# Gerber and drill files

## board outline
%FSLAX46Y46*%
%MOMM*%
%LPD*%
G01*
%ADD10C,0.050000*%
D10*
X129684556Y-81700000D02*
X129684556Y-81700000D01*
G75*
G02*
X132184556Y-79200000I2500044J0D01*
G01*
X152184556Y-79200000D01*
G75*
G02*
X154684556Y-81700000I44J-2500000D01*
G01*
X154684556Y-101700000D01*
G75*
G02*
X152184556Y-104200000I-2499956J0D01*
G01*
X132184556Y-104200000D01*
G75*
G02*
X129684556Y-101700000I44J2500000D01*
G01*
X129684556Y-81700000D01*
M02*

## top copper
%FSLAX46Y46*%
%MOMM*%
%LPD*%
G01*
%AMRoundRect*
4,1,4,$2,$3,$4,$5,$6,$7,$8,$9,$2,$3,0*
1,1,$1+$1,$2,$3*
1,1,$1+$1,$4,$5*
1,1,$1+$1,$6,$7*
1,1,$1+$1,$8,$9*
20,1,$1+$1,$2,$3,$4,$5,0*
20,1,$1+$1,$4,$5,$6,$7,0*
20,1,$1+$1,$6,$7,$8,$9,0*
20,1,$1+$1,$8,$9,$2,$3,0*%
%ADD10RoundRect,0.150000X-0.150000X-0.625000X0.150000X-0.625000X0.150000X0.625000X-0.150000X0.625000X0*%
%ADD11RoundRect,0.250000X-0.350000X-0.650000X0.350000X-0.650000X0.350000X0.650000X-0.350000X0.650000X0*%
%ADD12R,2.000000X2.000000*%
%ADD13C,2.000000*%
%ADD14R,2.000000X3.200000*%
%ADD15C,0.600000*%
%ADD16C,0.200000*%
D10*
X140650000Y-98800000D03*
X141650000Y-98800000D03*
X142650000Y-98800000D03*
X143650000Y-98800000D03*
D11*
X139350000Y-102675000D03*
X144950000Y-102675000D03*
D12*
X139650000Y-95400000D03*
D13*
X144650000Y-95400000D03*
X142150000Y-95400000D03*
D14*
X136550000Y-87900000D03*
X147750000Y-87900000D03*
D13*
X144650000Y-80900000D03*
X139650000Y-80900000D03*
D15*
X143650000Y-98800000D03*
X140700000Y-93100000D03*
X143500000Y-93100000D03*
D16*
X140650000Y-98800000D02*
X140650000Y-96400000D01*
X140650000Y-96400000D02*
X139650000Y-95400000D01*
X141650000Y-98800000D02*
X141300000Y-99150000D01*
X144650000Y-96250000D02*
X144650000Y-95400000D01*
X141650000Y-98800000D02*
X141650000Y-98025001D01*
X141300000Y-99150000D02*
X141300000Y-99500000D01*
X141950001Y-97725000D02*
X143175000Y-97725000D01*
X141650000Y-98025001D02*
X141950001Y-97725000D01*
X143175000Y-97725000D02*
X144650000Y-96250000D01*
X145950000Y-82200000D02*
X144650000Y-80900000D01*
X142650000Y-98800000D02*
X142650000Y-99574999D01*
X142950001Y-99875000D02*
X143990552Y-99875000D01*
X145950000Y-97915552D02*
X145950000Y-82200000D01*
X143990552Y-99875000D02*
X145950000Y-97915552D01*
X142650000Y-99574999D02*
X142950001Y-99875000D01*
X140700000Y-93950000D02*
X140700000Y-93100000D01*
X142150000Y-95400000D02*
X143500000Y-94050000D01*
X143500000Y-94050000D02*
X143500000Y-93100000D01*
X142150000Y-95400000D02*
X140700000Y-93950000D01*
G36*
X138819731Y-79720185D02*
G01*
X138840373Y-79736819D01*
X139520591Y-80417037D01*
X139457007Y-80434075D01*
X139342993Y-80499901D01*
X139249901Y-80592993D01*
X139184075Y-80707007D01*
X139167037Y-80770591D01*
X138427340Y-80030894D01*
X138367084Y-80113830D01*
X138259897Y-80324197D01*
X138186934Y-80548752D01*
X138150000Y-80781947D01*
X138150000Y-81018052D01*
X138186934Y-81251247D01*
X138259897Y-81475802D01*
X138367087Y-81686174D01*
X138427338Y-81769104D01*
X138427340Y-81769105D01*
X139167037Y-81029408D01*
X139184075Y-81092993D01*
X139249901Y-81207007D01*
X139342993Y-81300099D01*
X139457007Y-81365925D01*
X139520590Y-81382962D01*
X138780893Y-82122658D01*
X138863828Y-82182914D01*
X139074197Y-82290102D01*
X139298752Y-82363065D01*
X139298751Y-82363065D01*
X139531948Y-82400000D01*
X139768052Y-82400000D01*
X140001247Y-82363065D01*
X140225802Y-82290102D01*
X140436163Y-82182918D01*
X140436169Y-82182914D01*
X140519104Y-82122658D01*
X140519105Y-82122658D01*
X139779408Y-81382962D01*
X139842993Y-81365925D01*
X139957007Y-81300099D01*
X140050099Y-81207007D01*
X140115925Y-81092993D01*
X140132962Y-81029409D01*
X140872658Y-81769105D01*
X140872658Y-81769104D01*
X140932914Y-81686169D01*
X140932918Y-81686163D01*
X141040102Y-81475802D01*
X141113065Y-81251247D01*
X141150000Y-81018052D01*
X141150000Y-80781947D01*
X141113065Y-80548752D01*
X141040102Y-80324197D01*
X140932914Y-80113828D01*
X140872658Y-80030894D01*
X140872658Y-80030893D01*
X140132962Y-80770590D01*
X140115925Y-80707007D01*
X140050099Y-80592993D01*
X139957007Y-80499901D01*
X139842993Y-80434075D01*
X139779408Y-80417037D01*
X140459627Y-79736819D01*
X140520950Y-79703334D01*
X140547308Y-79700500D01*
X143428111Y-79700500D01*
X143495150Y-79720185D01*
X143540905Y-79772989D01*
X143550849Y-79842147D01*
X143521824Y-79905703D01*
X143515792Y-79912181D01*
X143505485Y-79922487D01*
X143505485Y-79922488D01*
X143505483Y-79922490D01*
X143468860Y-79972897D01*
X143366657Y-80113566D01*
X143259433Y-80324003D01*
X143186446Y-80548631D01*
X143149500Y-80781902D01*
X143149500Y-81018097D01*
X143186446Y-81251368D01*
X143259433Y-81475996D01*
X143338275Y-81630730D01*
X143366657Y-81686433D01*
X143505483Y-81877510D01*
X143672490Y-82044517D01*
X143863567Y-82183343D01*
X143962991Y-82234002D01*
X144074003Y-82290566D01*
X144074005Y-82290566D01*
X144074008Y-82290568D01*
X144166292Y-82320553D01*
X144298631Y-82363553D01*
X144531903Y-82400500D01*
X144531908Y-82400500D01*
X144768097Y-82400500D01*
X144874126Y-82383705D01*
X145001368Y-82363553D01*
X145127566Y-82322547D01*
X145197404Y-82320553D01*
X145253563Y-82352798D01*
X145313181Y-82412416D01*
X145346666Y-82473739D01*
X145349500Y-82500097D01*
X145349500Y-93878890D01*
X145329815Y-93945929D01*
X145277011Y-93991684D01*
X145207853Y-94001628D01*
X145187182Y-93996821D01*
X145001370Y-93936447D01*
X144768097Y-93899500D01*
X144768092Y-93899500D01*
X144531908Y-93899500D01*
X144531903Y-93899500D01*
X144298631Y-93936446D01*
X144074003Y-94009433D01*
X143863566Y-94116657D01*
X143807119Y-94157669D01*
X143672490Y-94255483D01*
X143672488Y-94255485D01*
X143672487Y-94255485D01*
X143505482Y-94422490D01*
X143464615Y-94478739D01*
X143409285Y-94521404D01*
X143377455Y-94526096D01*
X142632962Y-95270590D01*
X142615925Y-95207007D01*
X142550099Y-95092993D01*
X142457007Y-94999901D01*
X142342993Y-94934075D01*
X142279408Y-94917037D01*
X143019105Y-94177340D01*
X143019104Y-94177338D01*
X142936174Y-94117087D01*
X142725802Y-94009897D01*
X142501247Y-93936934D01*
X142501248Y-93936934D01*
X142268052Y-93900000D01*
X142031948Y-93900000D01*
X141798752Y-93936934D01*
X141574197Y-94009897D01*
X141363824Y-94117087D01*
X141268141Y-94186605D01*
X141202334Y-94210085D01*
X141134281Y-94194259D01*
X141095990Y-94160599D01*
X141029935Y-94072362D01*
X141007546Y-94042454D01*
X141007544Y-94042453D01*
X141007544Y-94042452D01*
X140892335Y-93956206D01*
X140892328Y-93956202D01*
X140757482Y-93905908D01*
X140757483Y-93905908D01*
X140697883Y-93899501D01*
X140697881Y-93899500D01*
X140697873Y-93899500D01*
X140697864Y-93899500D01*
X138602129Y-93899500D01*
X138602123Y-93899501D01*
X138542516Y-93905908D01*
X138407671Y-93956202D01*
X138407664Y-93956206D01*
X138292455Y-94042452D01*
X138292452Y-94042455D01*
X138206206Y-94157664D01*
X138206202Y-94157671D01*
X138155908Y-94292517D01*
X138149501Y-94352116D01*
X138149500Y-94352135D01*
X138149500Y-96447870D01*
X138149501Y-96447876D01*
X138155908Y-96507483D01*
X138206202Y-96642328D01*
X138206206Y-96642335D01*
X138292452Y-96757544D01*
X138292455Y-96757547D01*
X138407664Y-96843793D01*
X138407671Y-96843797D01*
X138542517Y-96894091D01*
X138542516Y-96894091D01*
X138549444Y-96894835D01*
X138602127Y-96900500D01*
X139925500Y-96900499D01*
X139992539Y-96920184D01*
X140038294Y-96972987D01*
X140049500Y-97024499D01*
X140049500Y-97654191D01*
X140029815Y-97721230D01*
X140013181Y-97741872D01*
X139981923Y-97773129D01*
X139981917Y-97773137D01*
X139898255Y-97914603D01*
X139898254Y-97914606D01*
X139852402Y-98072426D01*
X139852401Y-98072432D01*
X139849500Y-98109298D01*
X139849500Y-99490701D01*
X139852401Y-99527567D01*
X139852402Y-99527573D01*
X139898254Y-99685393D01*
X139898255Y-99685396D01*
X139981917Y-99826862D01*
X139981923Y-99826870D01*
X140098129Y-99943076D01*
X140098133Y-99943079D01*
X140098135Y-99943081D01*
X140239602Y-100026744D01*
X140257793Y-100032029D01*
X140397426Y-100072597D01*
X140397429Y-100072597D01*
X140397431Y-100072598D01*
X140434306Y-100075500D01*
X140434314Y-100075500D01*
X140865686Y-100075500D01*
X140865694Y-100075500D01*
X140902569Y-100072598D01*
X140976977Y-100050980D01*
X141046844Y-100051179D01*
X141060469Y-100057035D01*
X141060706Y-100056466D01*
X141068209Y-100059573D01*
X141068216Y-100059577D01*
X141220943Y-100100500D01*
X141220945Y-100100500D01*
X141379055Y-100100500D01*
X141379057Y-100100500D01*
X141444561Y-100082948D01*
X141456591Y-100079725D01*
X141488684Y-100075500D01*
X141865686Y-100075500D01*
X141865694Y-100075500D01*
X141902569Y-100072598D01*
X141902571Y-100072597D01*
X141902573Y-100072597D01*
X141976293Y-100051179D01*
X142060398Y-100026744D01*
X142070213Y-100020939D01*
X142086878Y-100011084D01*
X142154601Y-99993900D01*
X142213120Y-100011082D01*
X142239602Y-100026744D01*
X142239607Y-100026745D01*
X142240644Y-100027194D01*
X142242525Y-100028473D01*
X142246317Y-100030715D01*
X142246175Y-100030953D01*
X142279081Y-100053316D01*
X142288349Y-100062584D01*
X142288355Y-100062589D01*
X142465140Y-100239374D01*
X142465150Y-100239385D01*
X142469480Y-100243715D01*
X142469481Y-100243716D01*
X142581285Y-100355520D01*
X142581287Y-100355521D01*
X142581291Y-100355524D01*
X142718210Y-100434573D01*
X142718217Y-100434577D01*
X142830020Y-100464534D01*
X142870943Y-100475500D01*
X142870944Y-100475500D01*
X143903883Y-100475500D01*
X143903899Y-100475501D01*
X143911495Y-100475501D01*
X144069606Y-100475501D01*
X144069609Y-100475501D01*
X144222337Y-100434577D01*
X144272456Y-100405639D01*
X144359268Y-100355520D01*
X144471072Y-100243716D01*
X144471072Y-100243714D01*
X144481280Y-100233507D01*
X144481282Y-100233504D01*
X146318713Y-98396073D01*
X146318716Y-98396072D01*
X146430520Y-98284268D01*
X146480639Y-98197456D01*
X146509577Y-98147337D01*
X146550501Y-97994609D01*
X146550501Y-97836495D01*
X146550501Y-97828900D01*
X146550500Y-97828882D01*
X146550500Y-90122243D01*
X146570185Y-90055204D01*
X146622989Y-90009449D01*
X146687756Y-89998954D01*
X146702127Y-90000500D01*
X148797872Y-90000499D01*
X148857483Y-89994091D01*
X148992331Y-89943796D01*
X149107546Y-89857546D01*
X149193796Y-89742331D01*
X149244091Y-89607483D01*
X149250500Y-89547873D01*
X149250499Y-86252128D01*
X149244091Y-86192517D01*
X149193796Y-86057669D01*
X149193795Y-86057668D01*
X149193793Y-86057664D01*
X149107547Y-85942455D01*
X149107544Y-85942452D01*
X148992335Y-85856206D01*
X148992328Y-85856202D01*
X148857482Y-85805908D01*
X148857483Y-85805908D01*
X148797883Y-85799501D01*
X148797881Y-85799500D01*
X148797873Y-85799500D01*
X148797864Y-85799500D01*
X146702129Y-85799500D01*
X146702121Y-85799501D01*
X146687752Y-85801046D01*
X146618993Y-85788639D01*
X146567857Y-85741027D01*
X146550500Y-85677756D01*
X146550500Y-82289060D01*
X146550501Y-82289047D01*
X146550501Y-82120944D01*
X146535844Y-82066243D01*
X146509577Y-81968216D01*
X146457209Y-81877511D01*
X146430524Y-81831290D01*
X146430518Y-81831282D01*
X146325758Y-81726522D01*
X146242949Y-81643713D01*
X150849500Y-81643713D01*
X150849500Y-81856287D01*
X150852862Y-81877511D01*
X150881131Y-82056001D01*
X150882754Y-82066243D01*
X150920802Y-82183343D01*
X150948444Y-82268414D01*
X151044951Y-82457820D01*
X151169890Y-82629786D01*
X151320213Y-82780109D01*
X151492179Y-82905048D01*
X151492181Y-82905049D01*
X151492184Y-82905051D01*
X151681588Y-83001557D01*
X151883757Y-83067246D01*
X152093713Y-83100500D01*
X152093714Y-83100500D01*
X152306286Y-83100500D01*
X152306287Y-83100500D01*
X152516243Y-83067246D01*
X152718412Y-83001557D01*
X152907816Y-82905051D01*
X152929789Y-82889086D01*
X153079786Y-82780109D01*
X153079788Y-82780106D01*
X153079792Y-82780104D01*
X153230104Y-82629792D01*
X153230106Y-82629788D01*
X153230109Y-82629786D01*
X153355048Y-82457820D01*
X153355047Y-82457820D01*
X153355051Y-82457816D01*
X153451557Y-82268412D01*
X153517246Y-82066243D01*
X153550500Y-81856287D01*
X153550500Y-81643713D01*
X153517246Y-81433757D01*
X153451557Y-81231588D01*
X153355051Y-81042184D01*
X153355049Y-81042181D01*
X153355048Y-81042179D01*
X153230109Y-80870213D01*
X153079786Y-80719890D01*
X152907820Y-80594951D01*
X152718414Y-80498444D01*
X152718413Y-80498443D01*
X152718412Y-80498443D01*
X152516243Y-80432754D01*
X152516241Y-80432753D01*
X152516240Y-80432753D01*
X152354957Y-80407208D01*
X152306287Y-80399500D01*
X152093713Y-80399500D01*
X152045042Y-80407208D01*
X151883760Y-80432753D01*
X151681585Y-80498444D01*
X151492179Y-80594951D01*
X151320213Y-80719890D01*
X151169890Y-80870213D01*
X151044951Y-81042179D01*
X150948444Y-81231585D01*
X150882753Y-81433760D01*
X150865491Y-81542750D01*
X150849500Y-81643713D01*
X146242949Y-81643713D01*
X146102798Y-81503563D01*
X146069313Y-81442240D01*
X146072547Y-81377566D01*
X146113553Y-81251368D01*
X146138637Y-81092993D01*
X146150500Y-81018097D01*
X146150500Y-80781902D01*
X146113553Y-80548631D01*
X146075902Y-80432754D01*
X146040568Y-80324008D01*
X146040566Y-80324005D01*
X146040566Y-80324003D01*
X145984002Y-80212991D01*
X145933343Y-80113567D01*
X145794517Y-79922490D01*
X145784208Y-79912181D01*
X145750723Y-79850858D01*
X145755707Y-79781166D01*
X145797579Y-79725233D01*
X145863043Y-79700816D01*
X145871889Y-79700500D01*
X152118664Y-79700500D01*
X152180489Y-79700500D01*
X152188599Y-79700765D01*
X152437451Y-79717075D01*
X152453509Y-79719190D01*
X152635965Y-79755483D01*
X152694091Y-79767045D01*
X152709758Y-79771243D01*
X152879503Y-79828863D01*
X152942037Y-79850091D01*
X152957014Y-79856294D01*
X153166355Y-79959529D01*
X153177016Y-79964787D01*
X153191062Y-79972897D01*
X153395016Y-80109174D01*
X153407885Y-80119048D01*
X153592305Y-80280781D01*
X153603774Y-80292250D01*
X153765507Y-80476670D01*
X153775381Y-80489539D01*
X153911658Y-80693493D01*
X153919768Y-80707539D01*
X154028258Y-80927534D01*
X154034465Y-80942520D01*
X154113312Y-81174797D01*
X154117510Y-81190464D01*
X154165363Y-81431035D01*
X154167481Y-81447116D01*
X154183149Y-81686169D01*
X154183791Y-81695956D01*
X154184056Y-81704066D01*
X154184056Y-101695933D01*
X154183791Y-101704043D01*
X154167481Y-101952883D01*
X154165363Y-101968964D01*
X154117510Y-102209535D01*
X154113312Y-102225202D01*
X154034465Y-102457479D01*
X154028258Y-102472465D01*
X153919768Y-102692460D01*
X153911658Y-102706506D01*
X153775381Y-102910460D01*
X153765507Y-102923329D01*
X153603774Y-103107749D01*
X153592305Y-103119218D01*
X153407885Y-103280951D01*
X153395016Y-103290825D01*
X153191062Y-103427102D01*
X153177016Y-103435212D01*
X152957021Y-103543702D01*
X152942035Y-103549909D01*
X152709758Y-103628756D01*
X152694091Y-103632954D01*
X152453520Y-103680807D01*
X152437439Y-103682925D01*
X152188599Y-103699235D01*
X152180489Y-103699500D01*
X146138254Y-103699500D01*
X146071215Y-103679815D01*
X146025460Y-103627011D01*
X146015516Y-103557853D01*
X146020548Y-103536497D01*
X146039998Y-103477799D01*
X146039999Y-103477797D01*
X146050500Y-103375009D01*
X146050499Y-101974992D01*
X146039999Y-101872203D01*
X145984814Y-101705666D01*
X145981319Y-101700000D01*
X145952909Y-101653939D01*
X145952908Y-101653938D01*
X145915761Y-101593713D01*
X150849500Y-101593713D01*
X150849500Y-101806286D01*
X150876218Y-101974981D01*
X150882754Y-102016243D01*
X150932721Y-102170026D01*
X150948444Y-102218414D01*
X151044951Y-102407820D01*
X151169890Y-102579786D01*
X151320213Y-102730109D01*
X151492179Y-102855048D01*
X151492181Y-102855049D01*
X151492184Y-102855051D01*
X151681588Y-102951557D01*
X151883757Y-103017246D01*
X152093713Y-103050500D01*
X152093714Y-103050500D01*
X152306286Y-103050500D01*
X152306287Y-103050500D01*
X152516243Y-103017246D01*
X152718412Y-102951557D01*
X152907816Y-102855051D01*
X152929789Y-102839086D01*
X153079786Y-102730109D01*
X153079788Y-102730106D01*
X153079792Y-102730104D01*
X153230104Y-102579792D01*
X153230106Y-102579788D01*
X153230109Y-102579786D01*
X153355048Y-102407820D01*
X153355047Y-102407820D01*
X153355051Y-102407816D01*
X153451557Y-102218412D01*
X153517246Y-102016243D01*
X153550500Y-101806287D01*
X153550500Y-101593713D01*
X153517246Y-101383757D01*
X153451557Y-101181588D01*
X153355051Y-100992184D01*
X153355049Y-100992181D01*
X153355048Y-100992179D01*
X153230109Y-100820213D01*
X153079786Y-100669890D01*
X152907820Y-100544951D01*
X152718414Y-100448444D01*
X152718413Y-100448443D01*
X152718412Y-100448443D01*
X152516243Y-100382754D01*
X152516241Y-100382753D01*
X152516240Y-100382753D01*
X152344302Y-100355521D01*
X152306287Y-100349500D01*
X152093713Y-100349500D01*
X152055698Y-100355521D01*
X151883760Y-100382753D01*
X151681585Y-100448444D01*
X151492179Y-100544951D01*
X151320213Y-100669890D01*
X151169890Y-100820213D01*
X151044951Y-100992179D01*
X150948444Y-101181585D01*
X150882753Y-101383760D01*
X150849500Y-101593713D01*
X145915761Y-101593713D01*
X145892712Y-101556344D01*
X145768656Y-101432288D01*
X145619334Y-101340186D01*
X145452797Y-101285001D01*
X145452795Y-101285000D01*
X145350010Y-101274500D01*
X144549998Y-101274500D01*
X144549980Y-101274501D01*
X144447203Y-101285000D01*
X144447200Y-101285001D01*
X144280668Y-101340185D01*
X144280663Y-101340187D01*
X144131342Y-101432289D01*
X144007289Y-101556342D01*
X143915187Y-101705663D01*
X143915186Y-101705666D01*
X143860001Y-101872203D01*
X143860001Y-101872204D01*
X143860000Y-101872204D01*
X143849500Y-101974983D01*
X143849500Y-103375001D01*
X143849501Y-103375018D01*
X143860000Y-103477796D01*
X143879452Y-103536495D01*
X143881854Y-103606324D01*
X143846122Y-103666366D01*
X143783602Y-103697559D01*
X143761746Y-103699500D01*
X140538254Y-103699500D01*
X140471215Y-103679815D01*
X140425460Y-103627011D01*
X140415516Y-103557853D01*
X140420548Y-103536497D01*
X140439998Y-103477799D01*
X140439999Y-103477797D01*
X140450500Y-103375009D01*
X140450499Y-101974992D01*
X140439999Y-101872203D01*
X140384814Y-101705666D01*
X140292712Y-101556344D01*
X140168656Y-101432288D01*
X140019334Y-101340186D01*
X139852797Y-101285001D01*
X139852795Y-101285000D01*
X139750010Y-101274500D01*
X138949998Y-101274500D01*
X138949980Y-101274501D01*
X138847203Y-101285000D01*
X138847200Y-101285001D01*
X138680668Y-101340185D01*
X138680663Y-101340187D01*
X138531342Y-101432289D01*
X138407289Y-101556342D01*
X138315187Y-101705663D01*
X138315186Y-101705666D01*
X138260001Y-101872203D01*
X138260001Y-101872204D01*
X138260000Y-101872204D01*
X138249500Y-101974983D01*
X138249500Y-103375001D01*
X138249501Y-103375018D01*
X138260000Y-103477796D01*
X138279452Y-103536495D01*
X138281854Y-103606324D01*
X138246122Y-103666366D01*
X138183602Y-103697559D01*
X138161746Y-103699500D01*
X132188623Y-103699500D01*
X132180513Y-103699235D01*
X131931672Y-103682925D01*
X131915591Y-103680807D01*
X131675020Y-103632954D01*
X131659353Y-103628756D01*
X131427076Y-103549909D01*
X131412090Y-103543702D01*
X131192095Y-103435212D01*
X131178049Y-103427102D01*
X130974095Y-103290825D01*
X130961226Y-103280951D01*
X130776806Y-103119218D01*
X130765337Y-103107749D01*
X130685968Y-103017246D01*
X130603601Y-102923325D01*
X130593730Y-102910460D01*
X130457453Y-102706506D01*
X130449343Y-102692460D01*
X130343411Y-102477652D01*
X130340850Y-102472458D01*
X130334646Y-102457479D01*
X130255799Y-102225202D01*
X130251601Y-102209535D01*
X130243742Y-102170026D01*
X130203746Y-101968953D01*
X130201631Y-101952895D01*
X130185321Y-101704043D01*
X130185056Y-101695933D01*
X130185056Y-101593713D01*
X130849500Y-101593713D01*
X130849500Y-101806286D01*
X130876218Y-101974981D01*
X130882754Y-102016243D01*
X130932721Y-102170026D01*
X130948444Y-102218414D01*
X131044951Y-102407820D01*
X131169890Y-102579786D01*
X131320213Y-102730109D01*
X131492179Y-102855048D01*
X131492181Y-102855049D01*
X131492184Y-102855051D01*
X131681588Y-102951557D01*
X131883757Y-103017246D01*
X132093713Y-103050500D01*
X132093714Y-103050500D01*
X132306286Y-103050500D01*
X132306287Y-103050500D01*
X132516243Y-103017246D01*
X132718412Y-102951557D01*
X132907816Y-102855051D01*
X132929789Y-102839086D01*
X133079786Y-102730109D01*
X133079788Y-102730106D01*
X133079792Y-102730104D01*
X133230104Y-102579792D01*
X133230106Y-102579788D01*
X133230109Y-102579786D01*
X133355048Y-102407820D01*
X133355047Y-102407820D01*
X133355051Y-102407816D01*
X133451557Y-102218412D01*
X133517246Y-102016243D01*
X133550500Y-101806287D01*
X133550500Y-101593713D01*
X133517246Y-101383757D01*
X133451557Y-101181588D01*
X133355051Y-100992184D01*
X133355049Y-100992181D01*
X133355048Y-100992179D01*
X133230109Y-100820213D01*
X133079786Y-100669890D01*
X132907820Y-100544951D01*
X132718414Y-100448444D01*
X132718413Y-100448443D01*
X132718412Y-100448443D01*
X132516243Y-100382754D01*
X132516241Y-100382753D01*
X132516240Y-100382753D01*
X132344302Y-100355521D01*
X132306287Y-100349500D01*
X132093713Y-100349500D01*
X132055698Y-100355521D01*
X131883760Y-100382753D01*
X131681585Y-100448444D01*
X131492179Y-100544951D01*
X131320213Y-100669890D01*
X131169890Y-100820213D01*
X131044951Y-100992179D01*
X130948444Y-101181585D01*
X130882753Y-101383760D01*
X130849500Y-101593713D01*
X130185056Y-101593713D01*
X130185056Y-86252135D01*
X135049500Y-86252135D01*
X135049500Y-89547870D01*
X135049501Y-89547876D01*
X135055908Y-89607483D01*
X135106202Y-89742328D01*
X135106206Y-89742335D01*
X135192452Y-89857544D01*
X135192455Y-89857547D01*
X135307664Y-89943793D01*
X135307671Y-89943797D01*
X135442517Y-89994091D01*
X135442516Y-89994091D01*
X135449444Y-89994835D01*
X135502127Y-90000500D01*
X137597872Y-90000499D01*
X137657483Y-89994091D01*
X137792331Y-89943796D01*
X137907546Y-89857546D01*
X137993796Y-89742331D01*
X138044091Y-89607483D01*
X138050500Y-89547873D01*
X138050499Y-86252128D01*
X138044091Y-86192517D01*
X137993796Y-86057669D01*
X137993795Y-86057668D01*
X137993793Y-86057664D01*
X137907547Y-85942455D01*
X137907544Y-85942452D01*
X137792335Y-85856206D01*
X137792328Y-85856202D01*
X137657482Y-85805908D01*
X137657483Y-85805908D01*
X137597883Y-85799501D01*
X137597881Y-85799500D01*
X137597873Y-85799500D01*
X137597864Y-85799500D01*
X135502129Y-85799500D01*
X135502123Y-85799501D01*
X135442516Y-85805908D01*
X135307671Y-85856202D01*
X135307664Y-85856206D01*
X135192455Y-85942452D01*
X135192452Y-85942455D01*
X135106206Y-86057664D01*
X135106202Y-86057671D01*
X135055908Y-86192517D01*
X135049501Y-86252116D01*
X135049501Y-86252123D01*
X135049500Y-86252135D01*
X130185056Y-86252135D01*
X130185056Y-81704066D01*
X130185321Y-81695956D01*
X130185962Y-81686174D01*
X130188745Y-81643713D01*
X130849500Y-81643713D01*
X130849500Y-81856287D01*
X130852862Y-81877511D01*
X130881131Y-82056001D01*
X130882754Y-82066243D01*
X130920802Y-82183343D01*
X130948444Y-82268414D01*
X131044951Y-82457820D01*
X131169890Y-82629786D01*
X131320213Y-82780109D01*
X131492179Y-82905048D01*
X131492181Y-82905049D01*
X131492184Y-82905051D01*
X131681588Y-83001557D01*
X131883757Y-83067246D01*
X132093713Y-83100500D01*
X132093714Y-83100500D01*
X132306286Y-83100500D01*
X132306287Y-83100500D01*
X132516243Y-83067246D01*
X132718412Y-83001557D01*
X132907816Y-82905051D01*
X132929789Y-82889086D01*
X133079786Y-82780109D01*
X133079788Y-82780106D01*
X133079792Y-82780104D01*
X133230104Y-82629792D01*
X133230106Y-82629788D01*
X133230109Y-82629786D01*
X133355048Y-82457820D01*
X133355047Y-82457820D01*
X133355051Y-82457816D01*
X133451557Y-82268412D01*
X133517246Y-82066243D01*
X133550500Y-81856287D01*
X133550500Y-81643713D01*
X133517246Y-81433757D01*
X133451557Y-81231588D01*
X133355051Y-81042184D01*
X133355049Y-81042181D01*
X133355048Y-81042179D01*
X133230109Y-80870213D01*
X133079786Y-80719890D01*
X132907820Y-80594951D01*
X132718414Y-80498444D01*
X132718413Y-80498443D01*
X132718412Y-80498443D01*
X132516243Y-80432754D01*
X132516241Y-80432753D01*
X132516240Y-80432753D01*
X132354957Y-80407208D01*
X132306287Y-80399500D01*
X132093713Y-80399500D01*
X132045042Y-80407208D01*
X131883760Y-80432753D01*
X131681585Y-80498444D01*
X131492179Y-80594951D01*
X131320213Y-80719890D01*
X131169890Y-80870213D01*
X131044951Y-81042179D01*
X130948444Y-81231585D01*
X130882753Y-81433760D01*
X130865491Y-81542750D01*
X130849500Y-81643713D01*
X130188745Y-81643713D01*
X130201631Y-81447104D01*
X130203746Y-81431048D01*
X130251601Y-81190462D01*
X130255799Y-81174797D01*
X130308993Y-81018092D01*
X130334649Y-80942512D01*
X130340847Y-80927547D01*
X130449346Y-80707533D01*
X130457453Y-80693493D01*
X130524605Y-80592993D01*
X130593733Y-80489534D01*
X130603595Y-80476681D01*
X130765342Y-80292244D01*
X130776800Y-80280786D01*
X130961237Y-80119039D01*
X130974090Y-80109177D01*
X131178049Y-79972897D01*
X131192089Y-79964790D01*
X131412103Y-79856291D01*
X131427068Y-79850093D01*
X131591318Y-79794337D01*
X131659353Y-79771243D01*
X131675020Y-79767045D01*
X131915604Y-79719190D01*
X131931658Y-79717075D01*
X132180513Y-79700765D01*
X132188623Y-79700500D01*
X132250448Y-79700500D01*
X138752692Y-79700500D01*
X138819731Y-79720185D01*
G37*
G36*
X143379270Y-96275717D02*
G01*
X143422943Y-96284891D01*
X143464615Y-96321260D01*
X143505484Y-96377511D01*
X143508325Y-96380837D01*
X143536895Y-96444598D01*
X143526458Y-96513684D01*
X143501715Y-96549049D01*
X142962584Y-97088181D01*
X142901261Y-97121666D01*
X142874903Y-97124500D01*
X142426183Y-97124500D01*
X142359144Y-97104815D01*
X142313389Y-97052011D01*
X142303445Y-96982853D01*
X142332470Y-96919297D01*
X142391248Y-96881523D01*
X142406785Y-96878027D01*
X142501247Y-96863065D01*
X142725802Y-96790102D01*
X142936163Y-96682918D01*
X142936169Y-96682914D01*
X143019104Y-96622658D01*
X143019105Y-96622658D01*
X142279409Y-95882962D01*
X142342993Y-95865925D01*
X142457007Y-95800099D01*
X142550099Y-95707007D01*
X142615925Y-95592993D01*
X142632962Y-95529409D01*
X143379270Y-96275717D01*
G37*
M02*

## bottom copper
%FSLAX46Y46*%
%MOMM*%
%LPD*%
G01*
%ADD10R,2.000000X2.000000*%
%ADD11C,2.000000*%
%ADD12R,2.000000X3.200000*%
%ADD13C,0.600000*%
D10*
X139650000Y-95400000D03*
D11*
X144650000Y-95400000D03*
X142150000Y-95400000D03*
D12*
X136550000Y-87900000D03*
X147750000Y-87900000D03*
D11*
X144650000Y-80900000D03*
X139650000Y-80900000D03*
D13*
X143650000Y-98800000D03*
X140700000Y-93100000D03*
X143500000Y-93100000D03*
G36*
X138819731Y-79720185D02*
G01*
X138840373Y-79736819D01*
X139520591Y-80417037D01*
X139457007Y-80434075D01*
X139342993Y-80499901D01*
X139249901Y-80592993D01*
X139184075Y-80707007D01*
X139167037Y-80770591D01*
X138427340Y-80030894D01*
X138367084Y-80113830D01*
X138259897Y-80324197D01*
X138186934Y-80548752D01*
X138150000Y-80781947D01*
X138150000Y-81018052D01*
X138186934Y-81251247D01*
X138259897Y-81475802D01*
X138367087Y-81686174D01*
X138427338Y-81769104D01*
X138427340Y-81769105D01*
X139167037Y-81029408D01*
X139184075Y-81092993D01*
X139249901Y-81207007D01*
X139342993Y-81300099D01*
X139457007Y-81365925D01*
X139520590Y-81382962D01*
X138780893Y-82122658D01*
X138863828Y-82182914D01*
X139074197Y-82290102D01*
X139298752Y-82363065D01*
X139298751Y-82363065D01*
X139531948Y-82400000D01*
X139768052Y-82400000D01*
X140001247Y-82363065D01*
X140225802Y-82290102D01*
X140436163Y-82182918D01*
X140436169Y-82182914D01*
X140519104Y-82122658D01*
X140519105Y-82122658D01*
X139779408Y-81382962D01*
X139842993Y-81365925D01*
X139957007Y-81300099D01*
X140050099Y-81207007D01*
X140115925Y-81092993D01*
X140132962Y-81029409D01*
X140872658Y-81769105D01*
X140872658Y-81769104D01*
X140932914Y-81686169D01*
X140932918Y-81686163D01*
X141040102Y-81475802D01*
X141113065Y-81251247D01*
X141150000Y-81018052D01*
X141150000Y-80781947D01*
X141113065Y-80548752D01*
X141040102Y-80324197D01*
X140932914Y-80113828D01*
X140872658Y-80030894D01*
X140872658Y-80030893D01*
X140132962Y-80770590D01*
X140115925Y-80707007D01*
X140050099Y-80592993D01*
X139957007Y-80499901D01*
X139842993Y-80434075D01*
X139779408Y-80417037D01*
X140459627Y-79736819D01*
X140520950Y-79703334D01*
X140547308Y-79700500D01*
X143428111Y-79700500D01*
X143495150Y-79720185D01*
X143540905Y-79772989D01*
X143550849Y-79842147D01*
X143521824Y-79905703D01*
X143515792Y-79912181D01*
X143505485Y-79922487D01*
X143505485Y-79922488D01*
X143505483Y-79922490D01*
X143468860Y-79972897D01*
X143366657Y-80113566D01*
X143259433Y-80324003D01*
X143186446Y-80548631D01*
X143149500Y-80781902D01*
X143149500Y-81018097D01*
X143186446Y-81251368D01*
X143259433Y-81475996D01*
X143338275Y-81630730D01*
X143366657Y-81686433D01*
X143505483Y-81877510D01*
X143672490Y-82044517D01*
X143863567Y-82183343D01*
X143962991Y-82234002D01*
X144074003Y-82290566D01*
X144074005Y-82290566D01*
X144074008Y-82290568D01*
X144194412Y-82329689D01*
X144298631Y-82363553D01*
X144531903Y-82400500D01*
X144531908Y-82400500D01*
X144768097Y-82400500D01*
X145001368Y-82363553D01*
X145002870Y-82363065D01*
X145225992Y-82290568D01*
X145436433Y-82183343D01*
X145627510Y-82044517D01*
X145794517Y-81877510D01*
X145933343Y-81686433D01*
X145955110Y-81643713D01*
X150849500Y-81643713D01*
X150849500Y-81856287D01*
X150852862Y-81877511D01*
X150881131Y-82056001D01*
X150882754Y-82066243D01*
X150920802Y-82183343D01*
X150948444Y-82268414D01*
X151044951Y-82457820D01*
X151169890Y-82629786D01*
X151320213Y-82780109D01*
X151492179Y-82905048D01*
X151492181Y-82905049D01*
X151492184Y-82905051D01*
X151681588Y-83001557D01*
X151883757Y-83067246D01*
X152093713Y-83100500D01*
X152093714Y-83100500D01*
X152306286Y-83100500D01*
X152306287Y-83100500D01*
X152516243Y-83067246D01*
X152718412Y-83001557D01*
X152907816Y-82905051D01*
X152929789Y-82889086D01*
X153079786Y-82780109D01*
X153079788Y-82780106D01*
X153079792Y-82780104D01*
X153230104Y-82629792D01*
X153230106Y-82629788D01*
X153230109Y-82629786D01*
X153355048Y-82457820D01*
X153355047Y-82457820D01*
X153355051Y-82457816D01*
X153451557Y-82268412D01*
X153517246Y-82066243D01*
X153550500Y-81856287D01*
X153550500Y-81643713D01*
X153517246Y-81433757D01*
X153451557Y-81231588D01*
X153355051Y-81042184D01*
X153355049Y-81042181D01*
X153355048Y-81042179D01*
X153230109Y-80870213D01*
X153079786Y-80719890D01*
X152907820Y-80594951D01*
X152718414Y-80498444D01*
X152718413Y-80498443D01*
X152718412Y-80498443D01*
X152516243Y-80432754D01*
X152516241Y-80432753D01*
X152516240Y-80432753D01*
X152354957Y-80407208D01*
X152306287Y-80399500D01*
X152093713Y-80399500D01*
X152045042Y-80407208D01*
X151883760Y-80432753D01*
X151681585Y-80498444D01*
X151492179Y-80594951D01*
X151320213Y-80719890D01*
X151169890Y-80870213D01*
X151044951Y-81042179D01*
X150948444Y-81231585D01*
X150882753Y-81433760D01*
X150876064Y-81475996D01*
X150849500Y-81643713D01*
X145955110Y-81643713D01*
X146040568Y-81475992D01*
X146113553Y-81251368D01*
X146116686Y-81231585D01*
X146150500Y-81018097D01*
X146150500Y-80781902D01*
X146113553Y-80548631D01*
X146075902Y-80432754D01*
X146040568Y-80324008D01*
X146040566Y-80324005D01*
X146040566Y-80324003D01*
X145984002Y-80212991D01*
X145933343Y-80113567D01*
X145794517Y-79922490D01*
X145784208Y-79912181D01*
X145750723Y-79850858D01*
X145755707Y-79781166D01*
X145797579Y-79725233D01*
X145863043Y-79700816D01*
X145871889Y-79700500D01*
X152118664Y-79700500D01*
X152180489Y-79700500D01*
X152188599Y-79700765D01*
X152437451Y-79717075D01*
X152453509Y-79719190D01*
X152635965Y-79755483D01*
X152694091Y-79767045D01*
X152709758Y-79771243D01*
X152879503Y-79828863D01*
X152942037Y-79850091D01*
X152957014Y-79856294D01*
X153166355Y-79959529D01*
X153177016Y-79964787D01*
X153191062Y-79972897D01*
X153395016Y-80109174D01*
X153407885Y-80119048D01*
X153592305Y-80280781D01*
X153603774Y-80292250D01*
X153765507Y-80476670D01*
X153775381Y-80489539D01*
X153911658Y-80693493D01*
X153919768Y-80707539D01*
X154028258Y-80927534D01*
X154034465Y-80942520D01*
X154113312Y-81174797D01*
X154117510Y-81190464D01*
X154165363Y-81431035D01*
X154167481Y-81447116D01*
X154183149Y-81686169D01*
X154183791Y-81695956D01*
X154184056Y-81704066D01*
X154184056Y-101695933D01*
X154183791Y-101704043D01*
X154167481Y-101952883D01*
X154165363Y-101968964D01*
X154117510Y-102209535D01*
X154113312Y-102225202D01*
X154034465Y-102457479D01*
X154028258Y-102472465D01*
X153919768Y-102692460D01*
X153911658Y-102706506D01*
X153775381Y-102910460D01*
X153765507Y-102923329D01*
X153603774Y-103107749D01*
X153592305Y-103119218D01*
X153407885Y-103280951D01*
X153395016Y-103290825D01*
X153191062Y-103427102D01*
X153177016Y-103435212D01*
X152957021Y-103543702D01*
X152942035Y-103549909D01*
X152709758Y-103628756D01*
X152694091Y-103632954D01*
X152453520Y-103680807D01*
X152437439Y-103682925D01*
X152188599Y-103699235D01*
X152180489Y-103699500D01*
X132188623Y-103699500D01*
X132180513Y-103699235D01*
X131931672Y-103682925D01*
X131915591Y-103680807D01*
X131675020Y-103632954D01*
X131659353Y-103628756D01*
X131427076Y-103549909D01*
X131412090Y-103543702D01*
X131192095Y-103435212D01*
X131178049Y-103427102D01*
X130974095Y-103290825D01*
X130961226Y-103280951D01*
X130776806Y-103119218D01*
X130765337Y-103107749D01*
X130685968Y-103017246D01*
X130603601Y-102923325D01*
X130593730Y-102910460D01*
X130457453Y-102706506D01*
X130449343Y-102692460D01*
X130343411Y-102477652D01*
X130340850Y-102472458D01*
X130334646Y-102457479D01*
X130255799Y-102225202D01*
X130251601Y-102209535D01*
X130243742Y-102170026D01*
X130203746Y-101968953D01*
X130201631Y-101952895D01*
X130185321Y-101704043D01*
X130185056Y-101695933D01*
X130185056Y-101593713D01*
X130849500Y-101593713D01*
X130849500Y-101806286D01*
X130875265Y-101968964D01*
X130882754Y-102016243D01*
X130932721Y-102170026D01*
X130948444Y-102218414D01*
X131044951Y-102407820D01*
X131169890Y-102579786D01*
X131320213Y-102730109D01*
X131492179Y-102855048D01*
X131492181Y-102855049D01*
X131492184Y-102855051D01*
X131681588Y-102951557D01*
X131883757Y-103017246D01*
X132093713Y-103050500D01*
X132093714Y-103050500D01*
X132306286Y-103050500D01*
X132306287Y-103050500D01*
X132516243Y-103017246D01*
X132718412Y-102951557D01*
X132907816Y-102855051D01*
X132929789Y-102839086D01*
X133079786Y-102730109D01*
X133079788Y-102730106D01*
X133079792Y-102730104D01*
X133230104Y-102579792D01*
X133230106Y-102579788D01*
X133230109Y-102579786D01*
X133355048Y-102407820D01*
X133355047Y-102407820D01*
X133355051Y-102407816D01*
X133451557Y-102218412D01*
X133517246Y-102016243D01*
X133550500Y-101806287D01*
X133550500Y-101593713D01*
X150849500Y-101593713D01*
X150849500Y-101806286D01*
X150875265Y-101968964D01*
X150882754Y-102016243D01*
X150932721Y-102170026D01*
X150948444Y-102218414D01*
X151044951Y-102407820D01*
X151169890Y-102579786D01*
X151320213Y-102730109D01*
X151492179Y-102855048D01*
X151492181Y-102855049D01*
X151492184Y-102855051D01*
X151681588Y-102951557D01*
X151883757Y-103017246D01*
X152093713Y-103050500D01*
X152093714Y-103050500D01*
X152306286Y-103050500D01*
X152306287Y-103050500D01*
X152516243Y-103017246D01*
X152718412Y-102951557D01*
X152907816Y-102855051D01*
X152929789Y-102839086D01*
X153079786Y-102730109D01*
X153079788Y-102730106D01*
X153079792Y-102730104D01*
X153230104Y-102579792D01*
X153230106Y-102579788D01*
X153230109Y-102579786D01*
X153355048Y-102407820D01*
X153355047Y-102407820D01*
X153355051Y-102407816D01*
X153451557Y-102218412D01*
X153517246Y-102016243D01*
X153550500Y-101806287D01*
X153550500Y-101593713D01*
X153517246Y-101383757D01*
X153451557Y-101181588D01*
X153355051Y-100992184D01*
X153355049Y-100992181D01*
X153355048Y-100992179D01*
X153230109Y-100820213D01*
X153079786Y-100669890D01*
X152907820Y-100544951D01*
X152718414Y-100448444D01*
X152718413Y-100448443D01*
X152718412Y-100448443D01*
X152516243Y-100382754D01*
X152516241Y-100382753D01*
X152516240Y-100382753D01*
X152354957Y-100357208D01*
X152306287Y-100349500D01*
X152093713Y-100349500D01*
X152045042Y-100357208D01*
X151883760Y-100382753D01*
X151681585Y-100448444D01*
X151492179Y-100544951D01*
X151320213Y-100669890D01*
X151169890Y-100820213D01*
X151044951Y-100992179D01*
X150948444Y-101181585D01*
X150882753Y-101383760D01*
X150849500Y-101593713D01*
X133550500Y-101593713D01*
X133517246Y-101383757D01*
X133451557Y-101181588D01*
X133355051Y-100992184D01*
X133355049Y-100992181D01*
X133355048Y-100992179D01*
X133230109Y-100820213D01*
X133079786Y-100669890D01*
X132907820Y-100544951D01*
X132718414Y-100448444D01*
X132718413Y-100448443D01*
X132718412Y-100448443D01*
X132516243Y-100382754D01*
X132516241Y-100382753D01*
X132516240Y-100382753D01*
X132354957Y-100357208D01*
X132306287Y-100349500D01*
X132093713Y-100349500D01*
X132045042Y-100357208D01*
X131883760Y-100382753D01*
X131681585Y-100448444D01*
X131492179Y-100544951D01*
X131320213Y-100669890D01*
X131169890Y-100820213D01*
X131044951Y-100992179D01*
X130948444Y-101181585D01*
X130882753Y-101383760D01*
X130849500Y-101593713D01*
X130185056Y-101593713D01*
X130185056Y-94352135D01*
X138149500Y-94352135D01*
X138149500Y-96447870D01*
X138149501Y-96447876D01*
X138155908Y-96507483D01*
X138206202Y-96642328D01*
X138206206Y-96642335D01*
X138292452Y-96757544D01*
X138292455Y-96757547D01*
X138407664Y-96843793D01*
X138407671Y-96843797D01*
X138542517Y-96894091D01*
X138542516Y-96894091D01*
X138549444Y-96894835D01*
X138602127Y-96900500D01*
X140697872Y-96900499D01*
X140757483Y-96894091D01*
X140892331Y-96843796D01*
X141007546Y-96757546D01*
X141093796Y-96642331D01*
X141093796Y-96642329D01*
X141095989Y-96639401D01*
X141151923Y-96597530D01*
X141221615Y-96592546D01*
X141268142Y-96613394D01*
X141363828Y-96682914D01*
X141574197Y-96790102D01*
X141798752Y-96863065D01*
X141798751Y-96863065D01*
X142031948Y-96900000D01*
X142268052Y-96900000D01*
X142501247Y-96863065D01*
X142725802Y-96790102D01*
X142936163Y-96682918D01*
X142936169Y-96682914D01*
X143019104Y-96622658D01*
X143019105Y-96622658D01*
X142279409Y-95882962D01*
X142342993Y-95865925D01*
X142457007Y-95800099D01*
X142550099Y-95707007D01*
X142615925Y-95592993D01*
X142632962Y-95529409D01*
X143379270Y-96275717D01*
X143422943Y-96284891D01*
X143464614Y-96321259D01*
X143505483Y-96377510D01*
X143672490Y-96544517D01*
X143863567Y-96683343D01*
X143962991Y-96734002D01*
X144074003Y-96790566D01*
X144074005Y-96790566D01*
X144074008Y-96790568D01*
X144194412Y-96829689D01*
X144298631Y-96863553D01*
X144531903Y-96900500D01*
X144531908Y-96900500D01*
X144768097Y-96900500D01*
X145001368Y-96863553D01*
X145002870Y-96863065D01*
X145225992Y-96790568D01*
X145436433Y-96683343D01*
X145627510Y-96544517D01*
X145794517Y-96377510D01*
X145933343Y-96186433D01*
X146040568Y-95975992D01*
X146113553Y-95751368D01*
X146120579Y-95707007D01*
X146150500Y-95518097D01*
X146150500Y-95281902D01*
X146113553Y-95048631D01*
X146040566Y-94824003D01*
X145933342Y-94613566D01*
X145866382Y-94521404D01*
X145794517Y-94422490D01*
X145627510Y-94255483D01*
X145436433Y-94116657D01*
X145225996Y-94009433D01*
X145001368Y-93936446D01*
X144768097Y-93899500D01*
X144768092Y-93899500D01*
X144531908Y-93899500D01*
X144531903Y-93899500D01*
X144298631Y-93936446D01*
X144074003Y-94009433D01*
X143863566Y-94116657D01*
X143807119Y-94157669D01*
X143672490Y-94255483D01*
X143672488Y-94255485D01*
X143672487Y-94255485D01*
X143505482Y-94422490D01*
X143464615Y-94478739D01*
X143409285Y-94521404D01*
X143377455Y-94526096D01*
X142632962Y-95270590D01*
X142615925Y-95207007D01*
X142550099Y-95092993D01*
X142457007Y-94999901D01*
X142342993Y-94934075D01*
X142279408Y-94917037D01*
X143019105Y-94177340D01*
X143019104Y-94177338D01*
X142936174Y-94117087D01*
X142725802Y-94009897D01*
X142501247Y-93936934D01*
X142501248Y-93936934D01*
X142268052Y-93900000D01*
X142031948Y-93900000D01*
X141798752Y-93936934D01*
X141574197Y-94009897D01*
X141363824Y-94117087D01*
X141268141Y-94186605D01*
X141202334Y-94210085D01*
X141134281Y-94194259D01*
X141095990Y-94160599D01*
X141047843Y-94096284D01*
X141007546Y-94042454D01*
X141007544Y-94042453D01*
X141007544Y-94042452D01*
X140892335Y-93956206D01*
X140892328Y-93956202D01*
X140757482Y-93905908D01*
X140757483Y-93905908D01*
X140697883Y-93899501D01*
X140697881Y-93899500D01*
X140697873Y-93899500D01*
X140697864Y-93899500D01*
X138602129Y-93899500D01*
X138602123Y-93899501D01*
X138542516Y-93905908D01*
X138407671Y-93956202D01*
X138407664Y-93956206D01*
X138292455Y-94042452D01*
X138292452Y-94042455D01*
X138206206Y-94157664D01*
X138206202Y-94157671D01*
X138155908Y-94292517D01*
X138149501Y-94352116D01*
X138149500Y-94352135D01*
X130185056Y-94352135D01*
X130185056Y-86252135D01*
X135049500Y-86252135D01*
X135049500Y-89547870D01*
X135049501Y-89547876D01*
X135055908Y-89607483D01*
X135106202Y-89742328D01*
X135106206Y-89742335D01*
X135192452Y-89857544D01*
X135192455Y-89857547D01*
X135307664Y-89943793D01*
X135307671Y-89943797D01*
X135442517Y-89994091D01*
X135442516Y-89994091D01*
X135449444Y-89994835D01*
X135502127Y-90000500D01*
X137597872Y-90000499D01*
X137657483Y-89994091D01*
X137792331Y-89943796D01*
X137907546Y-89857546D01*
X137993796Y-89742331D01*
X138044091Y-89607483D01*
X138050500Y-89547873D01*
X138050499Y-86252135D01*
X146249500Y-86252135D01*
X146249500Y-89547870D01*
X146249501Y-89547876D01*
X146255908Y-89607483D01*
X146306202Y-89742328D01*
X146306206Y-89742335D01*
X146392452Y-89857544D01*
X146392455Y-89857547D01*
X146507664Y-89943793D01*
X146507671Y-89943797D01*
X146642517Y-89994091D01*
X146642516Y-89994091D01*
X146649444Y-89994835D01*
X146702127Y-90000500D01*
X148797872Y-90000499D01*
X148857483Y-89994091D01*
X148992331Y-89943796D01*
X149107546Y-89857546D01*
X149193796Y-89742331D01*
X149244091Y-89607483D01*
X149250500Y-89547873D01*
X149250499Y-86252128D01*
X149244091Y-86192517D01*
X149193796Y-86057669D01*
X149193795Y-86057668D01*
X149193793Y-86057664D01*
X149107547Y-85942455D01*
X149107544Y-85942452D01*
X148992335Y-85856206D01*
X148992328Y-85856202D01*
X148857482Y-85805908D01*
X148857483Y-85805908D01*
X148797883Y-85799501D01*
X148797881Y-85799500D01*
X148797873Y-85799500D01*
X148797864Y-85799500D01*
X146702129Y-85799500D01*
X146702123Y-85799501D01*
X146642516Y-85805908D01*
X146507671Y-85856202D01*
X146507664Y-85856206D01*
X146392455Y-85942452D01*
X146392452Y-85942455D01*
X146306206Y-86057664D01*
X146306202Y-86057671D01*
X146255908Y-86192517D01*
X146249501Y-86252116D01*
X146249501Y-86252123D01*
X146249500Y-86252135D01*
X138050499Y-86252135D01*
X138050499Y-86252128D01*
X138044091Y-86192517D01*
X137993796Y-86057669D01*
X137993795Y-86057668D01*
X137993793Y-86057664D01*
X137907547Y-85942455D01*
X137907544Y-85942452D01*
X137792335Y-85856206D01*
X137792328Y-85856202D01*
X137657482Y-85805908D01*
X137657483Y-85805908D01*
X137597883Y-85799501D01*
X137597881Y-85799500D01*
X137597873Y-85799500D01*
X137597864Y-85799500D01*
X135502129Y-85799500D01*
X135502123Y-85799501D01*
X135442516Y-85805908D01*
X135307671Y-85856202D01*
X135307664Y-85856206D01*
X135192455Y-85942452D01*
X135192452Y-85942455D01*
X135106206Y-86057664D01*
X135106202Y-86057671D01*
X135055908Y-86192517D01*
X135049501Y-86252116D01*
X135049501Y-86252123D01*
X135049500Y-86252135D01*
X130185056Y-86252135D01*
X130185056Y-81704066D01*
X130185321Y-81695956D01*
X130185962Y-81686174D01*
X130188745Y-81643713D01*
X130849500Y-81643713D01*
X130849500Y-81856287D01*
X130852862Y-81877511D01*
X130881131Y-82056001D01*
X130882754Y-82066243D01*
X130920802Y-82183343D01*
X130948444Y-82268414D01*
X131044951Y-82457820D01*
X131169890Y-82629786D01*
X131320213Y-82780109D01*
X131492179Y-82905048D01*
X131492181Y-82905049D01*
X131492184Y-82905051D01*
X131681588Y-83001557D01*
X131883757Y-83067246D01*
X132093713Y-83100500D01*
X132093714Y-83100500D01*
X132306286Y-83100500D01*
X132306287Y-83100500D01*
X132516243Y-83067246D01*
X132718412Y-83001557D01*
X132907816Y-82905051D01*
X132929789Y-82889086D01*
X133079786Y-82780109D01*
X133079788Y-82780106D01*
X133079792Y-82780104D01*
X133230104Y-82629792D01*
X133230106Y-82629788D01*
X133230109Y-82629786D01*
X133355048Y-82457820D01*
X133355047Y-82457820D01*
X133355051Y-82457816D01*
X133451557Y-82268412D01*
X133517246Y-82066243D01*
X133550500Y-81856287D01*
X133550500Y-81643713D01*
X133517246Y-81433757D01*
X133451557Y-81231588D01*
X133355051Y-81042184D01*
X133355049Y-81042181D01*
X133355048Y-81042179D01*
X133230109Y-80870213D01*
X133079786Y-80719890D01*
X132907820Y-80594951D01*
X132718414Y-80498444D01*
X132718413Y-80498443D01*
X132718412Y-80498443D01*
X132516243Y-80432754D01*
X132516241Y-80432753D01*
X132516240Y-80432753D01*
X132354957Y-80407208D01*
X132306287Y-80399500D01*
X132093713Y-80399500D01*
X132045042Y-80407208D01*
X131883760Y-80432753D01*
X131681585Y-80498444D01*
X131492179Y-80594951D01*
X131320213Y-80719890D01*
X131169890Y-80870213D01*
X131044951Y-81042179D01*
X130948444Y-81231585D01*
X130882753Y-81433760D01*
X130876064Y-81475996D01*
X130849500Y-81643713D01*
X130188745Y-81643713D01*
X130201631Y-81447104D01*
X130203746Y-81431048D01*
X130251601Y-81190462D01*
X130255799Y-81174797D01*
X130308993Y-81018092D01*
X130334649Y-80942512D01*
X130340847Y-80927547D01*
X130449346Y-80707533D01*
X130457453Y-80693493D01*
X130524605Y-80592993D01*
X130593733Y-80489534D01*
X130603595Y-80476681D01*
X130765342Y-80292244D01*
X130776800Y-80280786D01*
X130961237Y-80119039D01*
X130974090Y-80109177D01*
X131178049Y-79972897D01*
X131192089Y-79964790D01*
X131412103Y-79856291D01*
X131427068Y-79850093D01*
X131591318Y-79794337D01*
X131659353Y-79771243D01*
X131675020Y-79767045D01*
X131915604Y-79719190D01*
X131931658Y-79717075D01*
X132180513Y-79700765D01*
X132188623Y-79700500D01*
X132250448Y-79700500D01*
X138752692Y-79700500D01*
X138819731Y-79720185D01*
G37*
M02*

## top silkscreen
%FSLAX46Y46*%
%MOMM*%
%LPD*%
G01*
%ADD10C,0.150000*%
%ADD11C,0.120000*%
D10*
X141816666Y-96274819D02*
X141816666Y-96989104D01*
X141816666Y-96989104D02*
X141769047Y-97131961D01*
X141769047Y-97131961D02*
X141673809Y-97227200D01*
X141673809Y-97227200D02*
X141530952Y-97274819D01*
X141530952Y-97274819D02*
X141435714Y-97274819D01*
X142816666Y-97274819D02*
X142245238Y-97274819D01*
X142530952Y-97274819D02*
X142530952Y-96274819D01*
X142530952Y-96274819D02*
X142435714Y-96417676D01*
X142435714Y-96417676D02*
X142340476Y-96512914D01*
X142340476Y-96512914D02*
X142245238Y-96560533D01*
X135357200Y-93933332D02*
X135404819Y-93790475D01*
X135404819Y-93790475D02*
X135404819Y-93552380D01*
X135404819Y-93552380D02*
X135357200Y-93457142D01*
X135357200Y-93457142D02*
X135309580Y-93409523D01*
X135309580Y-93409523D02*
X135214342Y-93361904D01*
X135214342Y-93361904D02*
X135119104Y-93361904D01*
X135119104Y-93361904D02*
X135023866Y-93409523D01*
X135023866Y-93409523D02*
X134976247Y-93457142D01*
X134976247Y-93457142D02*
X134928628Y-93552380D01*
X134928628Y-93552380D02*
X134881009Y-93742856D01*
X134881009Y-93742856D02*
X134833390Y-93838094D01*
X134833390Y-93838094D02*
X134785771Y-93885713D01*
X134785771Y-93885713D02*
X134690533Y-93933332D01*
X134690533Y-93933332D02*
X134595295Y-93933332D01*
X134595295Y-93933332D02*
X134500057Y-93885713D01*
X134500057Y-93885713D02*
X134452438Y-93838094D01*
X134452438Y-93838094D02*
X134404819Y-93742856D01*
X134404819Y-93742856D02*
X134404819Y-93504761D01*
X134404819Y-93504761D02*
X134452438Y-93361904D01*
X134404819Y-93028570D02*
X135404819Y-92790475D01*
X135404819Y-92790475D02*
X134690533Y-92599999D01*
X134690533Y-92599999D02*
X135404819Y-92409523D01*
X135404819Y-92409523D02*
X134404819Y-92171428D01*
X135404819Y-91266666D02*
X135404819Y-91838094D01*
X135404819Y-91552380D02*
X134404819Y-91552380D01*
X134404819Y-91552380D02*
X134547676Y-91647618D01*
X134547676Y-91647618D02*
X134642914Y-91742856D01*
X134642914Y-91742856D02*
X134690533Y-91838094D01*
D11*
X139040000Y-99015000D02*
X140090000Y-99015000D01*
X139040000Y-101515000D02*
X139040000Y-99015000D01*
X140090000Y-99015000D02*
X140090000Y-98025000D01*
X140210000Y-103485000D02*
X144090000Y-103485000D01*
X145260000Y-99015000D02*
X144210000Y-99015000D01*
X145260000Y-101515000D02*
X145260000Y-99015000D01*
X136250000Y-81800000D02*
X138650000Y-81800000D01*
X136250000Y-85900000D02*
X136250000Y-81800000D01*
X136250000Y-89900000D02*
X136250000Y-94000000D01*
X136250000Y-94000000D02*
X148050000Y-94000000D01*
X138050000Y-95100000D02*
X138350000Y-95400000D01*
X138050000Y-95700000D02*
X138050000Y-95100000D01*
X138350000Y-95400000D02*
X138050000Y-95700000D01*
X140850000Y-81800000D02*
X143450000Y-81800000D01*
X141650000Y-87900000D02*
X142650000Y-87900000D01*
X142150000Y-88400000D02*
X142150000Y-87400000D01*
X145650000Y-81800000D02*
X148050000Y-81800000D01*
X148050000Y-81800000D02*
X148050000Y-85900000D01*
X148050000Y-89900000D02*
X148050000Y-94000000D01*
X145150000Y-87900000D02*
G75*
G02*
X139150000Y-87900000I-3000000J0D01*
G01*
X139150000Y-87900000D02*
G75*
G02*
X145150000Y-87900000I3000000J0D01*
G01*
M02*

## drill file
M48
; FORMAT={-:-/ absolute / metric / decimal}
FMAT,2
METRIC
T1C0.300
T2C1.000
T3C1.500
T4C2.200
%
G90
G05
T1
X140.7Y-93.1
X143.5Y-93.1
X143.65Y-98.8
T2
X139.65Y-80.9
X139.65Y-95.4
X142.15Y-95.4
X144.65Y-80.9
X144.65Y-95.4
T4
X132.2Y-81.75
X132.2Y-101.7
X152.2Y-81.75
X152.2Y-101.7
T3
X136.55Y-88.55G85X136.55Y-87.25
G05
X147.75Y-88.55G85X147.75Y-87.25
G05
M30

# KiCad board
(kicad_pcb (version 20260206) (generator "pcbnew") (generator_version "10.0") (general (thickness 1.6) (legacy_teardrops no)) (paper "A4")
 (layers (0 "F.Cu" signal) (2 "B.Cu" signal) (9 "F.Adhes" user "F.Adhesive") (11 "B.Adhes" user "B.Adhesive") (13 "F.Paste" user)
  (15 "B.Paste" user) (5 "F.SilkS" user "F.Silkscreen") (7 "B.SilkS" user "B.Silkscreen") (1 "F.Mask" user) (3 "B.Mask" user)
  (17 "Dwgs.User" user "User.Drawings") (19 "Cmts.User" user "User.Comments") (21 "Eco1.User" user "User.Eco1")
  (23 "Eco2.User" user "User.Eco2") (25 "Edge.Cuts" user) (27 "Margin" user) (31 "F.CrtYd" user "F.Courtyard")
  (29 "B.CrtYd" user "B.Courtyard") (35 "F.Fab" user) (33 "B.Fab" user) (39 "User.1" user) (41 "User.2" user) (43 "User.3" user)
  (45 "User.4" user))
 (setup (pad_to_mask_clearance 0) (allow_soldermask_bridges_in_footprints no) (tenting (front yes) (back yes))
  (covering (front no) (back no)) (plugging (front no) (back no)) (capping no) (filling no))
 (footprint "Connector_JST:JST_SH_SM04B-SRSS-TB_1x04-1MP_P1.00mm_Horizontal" (layer "F.Cu") (at 142.15 100.8)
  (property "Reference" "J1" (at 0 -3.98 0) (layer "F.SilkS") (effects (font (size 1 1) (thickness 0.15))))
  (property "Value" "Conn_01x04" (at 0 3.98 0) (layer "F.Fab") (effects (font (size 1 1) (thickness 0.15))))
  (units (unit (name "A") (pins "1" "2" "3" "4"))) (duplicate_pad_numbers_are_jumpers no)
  (fp_line (start -3.11 -1.785) (end -2.06 -1.785) (stroke (width 0.12) (type solid)) (layer "F.SilkS"))
  (fp_line (start -3.11 0.715) (end -3.11 -1.785) (stroke (width 0.12) (type solid)) (layer "F.SilkS"))
  (fp_line (start -2.06 -1.785) (end -2.06 -2.775) (stroke (width 0.12) (type solid)) (layer "F.SilkS"))
  (fp_line (start -1.94 2.685) (end 1.94 2.685) (stroke (width 0.12) (type solid)) (layer "F.SilkS"))
  (fp_line (start 3.11 -1.785) (end 2.06 -1.785) (stroke (width 0.12) (type solid)) (layer "F.SilkS"))
  (fp_line (start 3.11 0.715) (end 3.11 -1.785) (stroke (width 0.12) (type solid)) (layer "F.SilkS"))
  (pad "1" smd roundrect (at -1.5 -2) (size 0.6 1.55) (layers "F.Cu" "F.Mask" "F.Paste") (roundrect_rratio 0.25) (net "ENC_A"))
  (pad "2" smd roundrect (at -0.5 -2) (size 0.6 1.55) (layers "F.Cu" "F.Mask" "F.Paste") (roundrect_rratio 0.25) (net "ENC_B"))
  (pad "3" smd roundrect (at 0.5 -2) (size 0.6 1.55) (layers "F.Cu" "F.Mask" "F.Paste") (roundrect_rratio 0.25) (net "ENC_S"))
  (pad "4" smd roundrect (at 1.5 -2) (size 0.6 1.55) (layers "F.Cu" "F.Mask" "F.Paste") (roundrect_rratio 0.25) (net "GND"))
  (pad "MP" smd roundrect (at -2.8 1.875) (size 1.2 1.8) (layers "F.Cu" "F.Mask" "F.Paste") (roundrect_rratio 0.208333))
  (pad "MP" smd roundrect (at 2.8 1.875) (size 1.2 1.8) (layers "F.Cu" "F.Mask" "F.Paste") (roundrect_rratio 0.208333)))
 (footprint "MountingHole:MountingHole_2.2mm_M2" (layer "F.Cu") (at 132.2 101.7)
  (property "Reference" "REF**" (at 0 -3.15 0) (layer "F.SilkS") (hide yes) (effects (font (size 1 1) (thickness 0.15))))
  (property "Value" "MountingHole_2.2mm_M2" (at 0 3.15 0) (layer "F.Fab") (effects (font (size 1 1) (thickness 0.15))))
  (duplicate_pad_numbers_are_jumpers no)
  (pad "" np_thru_hole circle (at 0 0) (size 2.2 2.2) (drill 2.2) (layers "*.Cu" "*.Mask")))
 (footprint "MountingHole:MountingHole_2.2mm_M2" (layer "F.Cu") (at 152.2 101.7)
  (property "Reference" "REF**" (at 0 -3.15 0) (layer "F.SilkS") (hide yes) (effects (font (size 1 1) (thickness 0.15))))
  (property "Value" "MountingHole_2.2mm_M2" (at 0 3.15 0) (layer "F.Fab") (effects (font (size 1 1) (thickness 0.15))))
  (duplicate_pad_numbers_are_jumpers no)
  (pad "" np_thru_hole circle (at 0 0) (size 2.2 2.2) (drill 2.2) (layers "*.Cu" "*.Mask")))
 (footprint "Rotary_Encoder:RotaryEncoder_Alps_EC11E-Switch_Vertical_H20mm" (layer "F.Cu") (at 139.65 95.4 90)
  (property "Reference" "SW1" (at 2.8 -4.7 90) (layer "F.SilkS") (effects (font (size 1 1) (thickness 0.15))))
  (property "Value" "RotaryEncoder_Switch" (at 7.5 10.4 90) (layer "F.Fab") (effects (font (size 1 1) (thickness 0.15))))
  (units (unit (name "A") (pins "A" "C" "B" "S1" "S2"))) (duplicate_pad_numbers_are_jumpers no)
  (fp_line (start 13.6 -3.4) (end 13.6 -1) (stroke (width 0.12) (type solid)) (layer "F.SilkS"))
  (fp_line (start 9.5 -3.4) (end 13.6 -3.4) (stroke (width 0.12) (type solid)) (layer "F.SilkS"))
  (fp_line (start 5.5 -3.4) (end 1.4 -3.4) (stroke (width 0.12) (type solid)) (layer "F.SilkS"))
  (fp_line (start 1.4 -3.4) (end 1.4 8.4) (stroke (width 0.12) (type solid)) (layer "F.SilkS"))
  (fp_line (start 0.3 -1.6) (end 0 -1.3) (stroke (width 0.12) (type solid)) (layer "F.SilkS"))
  (fp_line (start -0.3 -1.6) (end 0.3 -1.6) (stroke (width 0.12) (type solid)) (layer "F.SilkS"))
  (fp_line (start 0 -1.3) (end -0.3 -1.6) (stroke (width 0.12) (type solid)) (layer "F.SilkS"))
  (fp_line (start 13.6 1.2) (end 13.6 3.8) (stroke (width 0.12) (type solid)) (layer "F.SilkS"))
  (fp_line (start 7.5 2) (end 7.5 3) (stroke (width 0.12) (type solid)) (layer "F.SilkS"))
  (fp_line (start 7 2.5) (end 8 2.5) (stroke (width 0.12) (type solid)) (layer "F.SilkS"))
  (fp_line (start 13.6 6) (end 13.6 8.4) (stroke (width 0.12) (type solid)) (layer "F.SilkS"))
  (fp_line (start 13.6 8.4) (end 9.5 8.4) (stroke (width 0.12) (type solid)) (layer "F.SilkS"))
  (fp_line (start 5.5 8.4) (end 1.4 8.4) (stroke (width 0.12) (type solid)) (layer "F.SilkS"))
  (fp_circle (center 7.5 2.5) (end 10.5 2.5) (stroke (width 0.12) (type solid)) (fill no) (layer "F.SilkS"))
  (pad "A" thru_hole rect (at 0 0 90) (size 2 2) (drill 1) (layers "*.Cu" "*.Mask") (remove_unused_layers no) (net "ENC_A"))
  (pad "B" thru_hole circle (at 0 5 90) (size 2 2) (drill 1) (layers "*.Cu" "*.Mask") (remove_unused_layers no) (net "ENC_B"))
  (pad "C" thru_hole circle (at 0 2.5 90) (size 2 2) (drill 1) (layers "*.Cu" "*.Mask") (remove_unused_layers no) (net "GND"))
  (pad "MP" thru_hole rect (at 7.5 -3.1 90) (size 3.2 2) (drill oval 2.8 1.5) (layers "*.Cu" "*.Mask") (remove_unused_layers no))
  (pad "MP" thru_hole rect (at 7.5 8.1 90) (size 3.2 2) (drill oval 2.8 1.5) (layers "*.Cu" "*.Mask") (remove_unused_layers no))
  (pad "S1" thru_hole circle (at 14.5 5 90) (size 2 2) (drill 1) (layers "*.Cu" "*.Mask") (remove_unused_layers no) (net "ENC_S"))
  (pad "S2" thru_hole circle (at 14.5 0 90) (size 2 2) (drill 1) (layers "*.Cu" "*.Mask") (remove_unused_layers no) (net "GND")))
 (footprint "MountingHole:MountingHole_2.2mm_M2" (layer "F.Cu") (at 152.2 81.75)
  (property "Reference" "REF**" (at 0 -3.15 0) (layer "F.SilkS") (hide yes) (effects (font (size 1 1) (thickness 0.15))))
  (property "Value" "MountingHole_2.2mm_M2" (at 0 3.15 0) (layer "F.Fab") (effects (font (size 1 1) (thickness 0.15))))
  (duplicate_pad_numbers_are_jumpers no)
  (pad "" np_thru_hole circle (at 0 0) (size 2.2 2.2) (drill 2.2) (layers "*.Cu" "*.Mask")))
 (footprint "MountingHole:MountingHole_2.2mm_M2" (layer "F.Cu") (at 132.2 81.75)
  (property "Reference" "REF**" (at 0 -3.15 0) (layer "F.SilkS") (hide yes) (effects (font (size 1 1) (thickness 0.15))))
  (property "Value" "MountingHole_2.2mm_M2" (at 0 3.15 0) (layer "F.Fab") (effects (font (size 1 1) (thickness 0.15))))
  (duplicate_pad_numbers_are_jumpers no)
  (pad "" np_thru_hole circle (at 0 0) (size 2.2 2.2) (drill 2.2) (layers "*.Cu" "*.Mask")))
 (gr_rect (start 129.684556 79.2) (end 154.684556 104.2) (radius 2.5) (stroke (width 0.05) (type solid)) (fill no) (layer "Edge.Cuts"))
 (segment (start 140.65 98.8) (end 140.65 96.4) (width 0.2) (layer "F.Cu") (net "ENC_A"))
 (segment (start 140.65 96.4) (end 139.65 95.4) (width 0.2) (layer "F.Cu") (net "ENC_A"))
 (segment (start 141.65 98.8) (end 141.3 99.15) (width 0.2) (layer "F.Cu") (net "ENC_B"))
 (segment (start 144.65 96.25) (end 144.65 95.4) (width 0.2) (layer "F.Cu") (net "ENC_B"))
 (segment (start 141.65 98.8) (end 141.65 98.025001) (width 0.2) (layer "F.Cu") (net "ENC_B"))
 (segment (start 141.3 99.15) (end 141.3 99.5) (width 0.2) (layer "F.Cu") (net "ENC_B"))
 (segment (start 141.950001 97.725) (end 143.175 97.725) (width 0.2) (layer "F.Cu") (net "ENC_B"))
 (segment (start 141.65 98.025001) (end 141.950001 97.725) (width 0.2) (layer "F.Cu") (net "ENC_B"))
 (segment (start 143.175 97.725) (end 144.65 96.25) (width 0.2) (layer "F.Cu") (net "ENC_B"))
 (segment (start 145.95 82.2) (end 144.65 80.9) (width 0.2) (layer "F.Cu") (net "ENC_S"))
 (segment (start 142.65 98.8) (end 142.65 99.574999) (width 0.2) (layer "F.Cu") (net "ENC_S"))
 (segment (start 142.950001 99.875) (end 143.990552 99.875) (width 0.2) (layer "F.Cu") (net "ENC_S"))
 (segment (start 145.95 97.915552) (end 145.95 82.2) (width 0.2) (layer "F.Cu") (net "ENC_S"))
 (segment (start 143.990552 99.875) (end 145.95 97.915552) (width 0.2) (layer "F.Cu") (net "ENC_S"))
 (segment (start 142.65 99.574999) (end 142.950001 99.875) (width 0.2) (layer "F.Cu") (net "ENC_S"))
 (segment (start 140.7 93.95) (end 140.7 93.1) (width 0.2) (layer "F.Cu") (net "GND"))
 (segment (start 142.15 95.4) (end 143.5 94.05) (width 0.2) (layer "F.Cu") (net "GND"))
 (segment (start 143.5 94.05) (end 143.5 93.1) (width 0.2) (layer "F.Cu") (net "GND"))
 (segment (start 142.15 95.4) (end 140.7 93.95) (width 0.2) (layer "F.Cu") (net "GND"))
 (via (at 143.65 98.8) (size 0.6) (drill 0.3) (layers "F.Cu" "B.Cu") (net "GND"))
 (via (at 140.7 93.1) (size 0.6) (drill 0.3) (layers "F.Cu" "B.Cu") (free yes) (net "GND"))
 (via (at 143.5 93.1) (size 0.6) (drill 0.3) (layers "F.Cu" "B.Cu") (free yes) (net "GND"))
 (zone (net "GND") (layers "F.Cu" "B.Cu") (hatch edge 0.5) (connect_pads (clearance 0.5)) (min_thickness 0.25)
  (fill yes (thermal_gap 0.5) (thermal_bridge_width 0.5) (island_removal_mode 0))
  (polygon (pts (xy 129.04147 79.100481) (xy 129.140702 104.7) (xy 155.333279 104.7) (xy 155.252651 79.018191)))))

